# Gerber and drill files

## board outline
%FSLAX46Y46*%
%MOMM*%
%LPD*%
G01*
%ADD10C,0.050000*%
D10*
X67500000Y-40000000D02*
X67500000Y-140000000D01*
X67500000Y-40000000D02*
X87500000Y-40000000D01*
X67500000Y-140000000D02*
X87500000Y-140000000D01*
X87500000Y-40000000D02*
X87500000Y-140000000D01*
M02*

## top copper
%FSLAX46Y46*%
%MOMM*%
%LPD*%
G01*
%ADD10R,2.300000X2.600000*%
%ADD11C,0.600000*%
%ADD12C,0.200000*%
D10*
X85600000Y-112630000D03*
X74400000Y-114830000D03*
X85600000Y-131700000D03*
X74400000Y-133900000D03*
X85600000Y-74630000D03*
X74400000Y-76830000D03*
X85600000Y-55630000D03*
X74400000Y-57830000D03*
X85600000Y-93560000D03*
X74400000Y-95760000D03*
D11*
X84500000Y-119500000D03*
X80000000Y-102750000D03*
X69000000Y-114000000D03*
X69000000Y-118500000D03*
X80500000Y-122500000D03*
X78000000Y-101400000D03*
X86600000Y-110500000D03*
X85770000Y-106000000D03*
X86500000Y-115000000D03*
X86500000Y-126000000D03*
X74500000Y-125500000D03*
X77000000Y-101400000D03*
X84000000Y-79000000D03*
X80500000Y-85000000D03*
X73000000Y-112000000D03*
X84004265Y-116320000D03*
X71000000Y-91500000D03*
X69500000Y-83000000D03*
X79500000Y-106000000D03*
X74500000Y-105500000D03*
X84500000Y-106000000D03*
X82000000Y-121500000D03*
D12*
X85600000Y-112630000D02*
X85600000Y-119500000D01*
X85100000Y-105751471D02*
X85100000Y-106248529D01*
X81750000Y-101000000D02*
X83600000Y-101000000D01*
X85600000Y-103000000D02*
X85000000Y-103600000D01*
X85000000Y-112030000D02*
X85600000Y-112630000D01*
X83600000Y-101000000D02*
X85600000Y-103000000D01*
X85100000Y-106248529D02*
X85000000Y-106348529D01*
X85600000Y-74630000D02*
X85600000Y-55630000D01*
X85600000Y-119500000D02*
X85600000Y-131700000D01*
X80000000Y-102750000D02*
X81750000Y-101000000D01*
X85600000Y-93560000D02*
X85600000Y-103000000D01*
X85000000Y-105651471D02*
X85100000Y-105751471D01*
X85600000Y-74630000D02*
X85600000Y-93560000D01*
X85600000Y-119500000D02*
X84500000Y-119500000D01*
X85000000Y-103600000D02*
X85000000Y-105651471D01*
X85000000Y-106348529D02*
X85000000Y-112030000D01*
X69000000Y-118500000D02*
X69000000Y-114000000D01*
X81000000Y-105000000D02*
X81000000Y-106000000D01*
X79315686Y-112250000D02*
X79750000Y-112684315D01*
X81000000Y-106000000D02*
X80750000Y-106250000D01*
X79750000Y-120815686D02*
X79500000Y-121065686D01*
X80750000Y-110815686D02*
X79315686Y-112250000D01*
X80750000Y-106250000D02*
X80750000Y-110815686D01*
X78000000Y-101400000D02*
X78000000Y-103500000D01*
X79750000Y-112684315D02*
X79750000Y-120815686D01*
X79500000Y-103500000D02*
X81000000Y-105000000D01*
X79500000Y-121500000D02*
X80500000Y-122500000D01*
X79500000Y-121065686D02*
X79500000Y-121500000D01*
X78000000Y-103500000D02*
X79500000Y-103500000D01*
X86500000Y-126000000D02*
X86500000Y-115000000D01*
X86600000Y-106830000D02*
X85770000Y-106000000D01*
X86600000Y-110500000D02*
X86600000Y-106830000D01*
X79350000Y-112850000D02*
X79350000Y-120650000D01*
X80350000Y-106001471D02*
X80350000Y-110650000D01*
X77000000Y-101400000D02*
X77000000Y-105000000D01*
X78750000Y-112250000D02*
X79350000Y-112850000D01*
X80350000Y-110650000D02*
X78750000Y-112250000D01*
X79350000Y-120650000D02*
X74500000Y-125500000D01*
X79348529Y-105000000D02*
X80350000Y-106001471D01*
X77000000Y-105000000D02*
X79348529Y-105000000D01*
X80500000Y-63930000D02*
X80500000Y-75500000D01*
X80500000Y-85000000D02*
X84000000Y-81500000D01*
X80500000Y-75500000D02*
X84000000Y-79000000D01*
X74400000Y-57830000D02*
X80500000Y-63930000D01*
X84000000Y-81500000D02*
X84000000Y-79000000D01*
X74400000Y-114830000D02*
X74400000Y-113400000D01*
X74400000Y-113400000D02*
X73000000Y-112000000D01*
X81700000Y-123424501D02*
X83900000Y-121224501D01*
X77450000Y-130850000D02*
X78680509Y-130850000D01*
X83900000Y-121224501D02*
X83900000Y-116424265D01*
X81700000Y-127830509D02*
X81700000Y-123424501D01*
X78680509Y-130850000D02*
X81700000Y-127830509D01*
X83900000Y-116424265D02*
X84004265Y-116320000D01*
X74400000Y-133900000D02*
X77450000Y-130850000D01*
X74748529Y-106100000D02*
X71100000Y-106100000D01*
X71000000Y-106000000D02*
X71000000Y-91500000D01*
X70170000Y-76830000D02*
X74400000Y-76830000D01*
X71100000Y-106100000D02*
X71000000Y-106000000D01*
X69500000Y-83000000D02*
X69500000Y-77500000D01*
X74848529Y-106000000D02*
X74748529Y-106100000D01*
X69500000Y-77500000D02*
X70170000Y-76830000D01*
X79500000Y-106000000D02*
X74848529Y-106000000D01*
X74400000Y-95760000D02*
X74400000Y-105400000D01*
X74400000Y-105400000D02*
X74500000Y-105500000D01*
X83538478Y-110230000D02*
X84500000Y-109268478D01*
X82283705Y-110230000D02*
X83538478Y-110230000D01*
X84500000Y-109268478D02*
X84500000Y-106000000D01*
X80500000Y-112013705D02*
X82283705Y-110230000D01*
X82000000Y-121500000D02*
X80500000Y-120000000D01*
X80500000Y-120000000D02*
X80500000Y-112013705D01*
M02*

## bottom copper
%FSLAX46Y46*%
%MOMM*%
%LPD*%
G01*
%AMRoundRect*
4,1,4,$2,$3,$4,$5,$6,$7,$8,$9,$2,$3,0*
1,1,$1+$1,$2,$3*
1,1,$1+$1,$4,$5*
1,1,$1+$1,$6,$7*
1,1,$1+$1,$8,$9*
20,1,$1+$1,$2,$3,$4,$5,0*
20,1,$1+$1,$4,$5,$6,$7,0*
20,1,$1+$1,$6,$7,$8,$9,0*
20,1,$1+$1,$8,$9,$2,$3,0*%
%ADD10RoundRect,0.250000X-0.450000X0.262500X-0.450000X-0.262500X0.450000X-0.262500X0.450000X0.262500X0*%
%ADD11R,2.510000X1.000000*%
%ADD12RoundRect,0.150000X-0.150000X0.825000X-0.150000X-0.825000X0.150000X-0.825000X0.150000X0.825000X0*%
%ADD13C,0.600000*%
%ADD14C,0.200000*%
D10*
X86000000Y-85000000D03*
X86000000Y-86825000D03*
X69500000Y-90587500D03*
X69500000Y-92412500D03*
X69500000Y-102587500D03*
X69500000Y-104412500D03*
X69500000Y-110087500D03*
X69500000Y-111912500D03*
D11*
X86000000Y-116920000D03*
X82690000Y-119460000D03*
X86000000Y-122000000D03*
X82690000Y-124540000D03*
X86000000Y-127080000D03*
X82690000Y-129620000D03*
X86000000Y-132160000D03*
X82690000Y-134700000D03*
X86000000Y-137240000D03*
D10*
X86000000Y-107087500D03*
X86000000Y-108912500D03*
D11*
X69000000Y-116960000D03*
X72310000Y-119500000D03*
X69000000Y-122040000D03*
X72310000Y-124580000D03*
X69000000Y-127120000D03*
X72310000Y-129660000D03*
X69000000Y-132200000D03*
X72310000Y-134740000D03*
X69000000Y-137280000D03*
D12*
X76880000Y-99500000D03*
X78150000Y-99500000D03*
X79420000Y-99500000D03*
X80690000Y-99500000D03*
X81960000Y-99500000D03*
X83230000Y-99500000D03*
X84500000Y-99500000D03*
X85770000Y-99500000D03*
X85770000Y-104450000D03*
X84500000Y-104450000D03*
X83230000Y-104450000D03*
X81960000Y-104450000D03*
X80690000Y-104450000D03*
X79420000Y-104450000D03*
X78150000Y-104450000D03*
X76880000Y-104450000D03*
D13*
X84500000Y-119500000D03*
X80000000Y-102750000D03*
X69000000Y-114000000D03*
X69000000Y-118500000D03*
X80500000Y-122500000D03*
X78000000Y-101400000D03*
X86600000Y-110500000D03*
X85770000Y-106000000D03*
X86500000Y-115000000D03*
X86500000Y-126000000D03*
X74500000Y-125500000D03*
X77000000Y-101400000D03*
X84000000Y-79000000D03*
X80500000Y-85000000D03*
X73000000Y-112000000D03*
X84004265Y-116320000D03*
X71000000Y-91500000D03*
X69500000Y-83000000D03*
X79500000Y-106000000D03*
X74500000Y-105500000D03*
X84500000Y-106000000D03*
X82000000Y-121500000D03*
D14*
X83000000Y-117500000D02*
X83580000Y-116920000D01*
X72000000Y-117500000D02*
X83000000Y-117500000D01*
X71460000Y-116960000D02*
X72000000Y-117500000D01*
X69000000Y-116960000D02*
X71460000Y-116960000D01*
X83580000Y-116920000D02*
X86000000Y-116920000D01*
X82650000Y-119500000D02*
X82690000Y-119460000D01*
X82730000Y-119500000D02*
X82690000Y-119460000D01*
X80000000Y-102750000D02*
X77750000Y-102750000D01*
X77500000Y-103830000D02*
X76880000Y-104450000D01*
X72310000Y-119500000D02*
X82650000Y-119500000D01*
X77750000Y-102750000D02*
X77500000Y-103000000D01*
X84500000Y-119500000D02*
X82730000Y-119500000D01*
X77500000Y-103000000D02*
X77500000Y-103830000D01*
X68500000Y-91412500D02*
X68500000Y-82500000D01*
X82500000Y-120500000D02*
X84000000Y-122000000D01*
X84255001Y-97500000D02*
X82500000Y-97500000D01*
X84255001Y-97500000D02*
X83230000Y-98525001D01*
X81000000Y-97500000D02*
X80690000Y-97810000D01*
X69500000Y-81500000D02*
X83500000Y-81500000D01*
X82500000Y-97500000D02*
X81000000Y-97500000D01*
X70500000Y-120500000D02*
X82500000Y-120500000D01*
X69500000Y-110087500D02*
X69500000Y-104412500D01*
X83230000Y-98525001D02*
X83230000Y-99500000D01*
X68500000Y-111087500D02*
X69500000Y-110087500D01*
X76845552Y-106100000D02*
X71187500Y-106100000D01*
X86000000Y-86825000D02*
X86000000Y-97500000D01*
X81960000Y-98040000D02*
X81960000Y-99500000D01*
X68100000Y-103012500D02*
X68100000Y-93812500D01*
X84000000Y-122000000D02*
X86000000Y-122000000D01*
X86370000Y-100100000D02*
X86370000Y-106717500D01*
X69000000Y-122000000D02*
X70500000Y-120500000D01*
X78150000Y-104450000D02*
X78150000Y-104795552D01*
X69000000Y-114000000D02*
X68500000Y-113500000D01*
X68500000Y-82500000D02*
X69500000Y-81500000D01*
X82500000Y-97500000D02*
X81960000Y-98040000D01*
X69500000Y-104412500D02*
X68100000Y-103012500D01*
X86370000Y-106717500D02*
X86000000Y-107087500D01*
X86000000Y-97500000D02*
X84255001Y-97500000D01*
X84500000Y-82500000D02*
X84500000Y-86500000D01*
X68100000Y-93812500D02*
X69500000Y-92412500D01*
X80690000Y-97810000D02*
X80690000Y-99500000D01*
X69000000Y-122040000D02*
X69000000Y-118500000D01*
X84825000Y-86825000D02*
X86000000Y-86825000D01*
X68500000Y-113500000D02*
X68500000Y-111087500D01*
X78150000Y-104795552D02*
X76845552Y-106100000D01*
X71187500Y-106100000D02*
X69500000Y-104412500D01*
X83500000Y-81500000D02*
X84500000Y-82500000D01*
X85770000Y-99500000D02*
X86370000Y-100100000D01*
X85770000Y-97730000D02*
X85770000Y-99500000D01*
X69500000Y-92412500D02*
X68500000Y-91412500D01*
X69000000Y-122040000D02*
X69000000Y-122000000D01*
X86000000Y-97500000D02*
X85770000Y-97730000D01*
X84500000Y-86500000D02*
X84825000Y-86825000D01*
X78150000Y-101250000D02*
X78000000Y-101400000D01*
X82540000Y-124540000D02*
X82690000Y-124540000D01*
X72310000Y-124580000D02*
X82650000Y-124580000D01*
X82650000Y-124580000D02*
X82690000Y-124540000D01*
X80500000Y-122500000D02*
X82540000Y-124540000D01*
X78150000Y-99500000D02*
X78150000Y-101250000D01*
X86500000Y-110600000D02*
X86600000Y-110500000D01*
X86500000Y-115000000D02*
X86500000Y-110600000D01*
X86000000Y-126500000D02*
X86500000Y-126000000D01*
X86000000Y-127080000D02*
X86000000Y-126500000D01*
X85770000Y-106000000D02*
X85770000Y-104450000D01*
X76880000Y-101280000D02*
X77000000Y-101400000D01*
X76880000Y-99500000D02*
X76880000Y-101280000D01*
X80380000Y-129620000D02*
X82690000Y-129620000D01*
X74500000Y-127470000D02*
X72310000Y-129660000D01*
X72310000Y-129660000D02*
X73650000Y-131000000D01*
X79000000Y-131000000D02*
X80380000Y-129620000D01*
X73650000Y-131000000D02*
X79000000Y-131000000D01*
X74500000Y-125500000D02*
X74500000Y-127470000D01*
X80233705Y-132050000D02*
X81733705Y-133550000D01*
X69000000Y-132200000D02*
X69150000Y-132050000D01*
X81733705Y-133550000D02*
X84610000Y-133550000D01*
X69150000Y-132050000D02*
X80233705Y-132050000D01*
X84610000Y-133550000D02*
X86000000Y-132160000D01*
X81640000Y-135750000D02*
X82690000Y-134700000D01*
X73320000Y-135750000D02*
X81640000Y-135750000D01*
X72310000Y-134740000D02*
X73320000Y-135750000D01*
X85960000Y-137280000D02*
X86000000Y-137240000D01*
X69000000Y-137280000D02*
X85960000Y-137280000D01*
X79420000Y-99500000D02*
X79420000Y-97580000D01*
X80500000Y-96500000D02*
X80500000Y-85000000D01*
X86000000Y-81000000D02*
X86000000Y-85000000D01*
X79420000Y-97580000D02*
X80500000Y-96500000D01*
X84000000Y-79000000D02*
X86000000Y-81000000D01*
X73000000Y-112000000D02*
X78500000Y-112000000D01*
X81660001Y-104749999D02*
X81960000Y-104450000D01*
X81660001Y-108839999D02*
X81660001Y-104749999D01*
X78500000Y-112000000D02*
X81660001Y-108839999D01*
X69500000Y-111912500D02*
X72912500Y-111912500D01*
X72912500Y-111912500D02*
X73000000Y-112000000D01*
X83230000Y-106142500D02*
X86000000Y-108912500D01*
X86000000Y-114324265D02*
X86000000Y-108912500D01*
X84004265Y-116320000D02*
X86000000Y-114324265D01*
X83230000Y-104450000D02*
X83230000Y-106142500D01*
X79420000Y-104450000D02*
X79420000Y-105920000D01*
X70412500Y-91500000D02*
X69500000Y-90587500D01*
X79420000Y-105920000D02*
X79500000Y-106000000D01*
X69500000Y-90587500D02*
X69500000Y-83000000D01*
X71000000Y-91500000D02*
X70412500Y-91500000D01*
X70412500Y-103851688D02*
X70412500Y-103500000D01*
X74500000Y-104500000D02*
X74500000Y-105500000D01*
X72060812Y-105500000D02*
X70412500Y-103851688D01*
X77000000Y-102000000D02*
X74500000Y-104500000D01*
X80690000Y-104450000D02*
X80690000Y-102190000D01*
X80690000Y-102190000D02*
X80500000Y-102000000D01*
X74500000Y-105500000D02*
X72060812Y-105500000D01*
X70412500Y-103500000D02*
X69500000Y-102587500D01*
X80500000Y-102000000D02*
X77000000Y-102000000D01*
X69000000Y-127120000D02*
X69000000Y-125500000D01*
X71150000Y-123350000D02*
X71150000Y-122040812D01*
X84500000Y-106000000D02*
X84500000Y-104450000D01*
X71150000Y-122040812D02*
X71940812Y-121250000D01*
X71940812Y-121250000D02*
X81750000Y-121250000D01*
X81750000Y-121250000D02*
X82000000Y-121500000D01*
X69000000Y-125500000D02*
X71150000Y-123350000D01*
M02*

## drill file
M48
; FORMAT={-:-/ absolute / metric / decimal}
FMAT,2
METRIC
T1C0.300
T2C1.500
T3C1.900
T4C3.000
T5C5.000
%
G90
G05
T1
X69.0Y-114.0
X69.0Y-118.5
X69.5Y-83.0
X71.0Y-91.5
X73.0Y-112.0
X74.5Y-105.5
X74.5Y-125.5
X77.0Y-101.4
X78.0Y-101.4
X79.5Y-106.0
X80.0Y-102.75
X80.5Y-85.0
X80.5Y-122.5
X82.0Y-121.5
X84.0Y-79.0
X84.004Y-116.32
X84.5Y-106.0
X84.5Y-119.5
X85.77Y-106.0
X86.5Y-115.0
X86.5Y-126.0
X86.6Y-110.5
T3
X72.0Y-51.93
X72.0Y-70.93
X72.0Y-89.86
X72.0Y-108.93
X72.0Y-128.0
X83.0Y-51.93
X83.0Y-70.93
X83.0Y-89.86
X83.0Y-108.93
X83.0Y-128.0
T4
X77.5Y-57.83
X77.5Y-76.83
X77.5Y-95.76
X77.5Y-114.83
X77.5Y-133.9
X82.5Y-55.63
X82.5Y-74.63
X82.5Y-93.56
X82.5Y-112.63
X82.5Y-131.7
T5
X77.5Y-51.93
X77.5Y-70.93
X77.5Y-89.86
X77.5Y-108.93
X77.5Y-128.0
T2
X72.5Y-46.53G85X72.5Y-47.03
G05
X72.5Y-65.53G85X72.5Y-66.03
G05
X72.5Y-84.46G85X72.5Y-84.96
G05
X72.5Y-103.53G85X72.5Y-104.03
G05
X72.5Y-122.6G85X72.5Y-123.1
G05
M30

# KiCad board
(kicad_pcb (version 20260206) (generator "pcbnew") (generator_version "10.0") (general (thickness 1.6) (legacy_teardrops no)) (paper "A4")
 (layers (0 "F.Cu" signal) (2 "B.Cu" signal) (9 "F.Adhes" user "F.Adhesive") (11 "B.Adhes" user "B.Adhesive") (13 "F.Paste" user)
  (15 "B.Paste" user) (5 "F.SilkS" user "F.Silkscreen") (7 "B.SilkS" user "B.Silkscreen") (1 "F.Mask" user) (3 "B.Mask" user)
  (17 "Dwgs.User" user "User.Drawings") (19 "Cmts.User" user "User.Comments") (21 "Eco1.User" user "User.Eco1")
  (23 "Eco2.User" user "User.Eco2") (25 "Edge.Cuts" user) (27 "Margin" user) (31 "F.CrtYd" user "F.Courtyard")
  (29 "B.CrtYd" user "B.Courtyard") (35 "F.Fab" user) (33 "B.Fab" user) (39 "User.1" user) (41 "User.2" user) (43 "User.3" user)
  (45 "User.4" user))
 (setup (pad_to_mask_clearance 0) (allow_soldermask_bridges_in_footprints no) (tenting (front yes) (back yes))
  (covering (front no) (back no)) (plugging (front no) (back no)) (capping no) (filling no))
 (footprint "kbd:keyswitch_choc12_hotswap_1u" (layer "F.Cu") (at 77.5 108.93)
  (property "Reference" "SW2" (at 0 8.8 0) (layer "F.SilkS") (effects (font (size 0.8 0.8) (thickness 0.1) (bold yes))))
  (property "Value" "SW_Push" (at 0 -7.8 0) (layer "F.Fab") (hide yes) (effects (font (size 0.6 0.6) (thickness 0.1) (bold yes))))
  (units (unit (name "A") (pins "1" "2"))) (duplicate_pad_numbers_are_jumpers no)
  (pad "" np_thru_hole circle (at -5.5 0 270) (size 1.9 1.9) (drill 1.9) (layers "*.Cu" "*.Mask"))
  (pad "" np_thru_hole oval (at -5 -5.15) (size 1.5 2) (drill oval 1.5 2) (layers "*.Cu" "*.Mask"))
  (pad "" np_thru_hole circle (at 0 0 270) (size 5 5) (drill 5) (layers "*.Cu" "*.Mask"))
  (pad "" np_thru_hole circle (at 0 5.9 270) (size 3 3) (drill 3) (layers "*.Cu" "*.Mask"))
  (pad "" np_thru_hole circle (at 5 3.7 270) (size 3 3) (drill 3) (layers "*.Cu" "*.Mask"))
  (pad "" np_thru_hole circle (at 5.5 0 270) (size 1.9 1.9) (drill 1.9) (layers "*.Cu" "*.Mask"))
  (pad "1" smd rect (at 8.1 3.7 180) (size 2.3 2.6) (layers "F.Cu" "F.Mask" "F.Paste") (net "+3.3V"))
  (pad "2" smd rect (at -3.1 5.9 180) (size 2.3 2.6) (layers "F.Cu" "F.Mask" "F.Paste") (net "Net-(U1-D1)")))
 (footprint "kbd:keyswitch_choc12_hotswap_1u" (layer "F.Cu") (at 77.5 128)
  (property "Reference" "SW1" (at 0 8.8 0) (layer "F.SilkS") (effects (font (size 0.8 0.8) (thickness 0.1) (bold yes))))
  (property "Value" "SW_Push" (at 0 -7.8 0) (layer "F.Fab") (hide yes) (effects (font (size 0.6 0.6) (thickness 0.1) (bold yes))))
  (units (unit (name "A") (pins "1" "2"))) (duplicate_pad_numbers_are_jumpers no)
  (pad "" np_thru_hole circle (at -5.5 0 270) (size 1.9 1.9) (drill 1.9) (layers "*.Cu" "*.Mask"))
  (pad "" np_thru_hole oval (at -5 -5.15) (size 1.5 2) (drill oval 1.5 2) (layers "*.Cu" "*.Mask"))
  (pad "" np_thru_hole circle (at 0 0 270) (size 5 5) (drill 5) (layers "*.Cu" "*.Mask"))
  (pad "" np_thru_hole circle (at 0 5.9 270) (size 3 3) (drill 3) (layers "*.Cu" "*.Mask"))
  (pad "" np_thru_hole circle (at 5 3.7 270) (size 3 3) (drill 3) (layers "*.Cu" "*.Mask"))
  (pad "" np_thru_hole circle (at 5.5 0 270) (size 1.9 1.9) (drill 1.9) (layers "*.Cu" "*.Mask"))
  (pad "1" smd rect (at 8.1 3.7 180) (size 2.3 2.6) (layers "F.Cu" "F.Mask" "F.Paste") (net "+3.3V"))
  (pad "2" smd rect (at -3.1 5.9 180) (size 2.3 2.6) (layers "F.Cu" "F.Mask" "F.Paste") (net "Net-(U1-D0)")))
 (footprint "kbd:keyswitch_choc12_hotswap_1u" (layer "F.Cu") (at 77.5 70.93)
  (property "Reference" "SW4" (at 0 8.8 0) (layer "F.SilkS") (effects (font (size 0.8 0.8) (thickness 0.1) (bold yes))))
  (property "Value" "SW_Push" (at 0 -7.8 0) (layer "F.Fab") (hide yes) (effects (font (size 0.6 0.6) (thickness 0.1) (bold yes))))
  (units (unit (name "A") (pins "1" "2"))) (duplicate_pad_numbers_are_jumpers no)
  (pad "" np_thru_hole circle (at -5.5 0 270) (size 1.9 1.9) (drill 1.9) (layers "*.Cu" "*.Mask"))
  (pad "" np_thru_hole oval (at -5 -5.15) (size 1.5 2) (drill oval 1.5 2) (layers "*.Cu" "*.Mask"))
  (pad "" np_thru_hole circle (at 0 0 270) (size 5 5) (drill 5) (layers "*.Cu" "*.Mask"))
  (pad "" np_thru_hole circle (at 0 5.9 270) (size 3 3) (drill 3) (layers "*.Cu" "*.Mask"))
  (pad "" np_thru_hole circle (at 5 3.7 270) (size 3 3) (drill 3) (layers "*.Cu" "*.Mask"))
  (pad "" np_thru_hole circle (at 5.5 0 270) (size 1.9 1.9) (drill 1.9) (layers "*.Cu" "*.Mask"))
  (pad "1" smd rect (at 8.1 3.7 180) (size 2.3 2.6) (layers "F.Cu" "F.Mask" "F.Paste") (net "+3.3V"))
  (pad "2" smd rect (at -3.1 5.9 180) (size 2.3 2.6) (layers "F.Cu" "F.Mask" "F.Paste") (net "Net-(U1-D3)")))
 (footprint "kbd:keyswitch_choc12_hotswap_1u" (layer "F.Cu") (at 77.5 51.93)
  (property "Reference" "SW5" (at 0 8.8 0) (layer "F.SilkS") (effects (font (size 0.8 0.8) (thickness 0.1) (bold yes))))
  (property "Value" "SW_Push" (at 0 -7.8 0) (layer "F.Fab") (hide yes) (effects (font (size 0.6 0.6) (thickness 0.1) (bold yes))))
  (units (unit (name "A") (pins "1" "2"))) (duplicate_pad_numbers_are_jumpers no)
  (pad "" np_thru_hole circle (at -5.5 0 270) (size 1.9 1.9) (drill 1.9) (layers "*.Cu" "*.Mask"))
  (pad "" np_thru_hole oval (at -5 -5.15) (size 1.5 2) (drill oval 1.5 2) (layers "*.Cu" "*.Mask"))
  (pad "" np_thru_hole circle (at 0 0 270) (size 5 5) (drill 5) (layers "*.Cu" "*.Mask"))
  (pad "" np_thru_hole circle (at 0 5.9 270) (size 3 3) (drill 3) (layers "*.Cu" "*.Mask"))
  (pad "" np_thru_hole circle (at 5 3.7 270) (size 3 3) (drill 3) (layers "*.Cu" "*.Mask"))
  (pad "" np_thru_hole circle (at 5.5 0 270) (size 1.9 1.9) (drill 1.9) (layers "*.Cu" "*.Mask"))
  (pad "1" smd rect (at 8.1 3.7 180) (size 2.3 2.6) (layers "F.Cu" "F.Mask" "F.Paste") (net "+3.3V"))
  (pad "2" smd rect (at -3.1 5.9 180) (size 2.3 2.6) (layers "F.Cu" "F.Mask" "F.Paste") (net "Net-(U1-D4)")))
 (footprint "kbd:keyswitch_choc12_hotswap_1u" (layer "F.Cu") (at 77.5 89.86)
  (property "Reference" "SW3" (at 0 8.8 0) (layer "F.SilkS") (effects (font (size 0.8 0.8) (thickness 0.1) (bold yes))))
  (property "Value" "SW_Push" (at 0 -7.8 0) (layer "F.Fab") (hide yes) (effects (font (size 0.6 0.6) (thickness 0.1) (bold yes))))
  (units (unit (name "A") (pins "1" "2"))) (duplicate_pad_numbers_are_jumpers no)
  (pad "" np_thru_hole circle (at -5.5 0 270) (size 1.9 1.9) (drill 1.9) (layers "*.Cu" "*.Mask"))
  (pad "" np_thru_hole oval (at -5 -5.15) (size 1.5 2) (drill oval 1.5 2) (layers "*.Cu" "*.Mask"))
  (pad "" np_thru_hole circle (at 0 0 270) (size 5 5) (drill 5) (layers "*.Cu" "*.Mask"))
  (pad "" np_thru_hole circle (at 0 5.9 270) (size 3 3) (drill 3) (layers "*.Cu" "*.Mask"))
  (pad "" np_thru_hole circle (at 5 3.7 270) (size 3 3) (drill 3) (layers "*.Cu" "*.Mask"))
  (pad "" np_thru_hole circle (at 5.5 0 270) (size 1.9 1.9) (drill 1.9) (layers "*.Cu" "*.Mask"))
  (pad "1" smd rect (at 8.1 3.7 180) (size 2.3 2.6) (layers "F.Cu" "F.Mask" "F.Paste") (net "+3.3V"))
  (pad "2" smd rect (at -3.1 5.9 180) (size 2.3 2.6) (layers "F.Cu" "F.Mask" "F.Paste") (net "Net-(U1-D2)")))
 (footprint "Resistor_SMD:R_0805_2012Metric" (layer "B.Cu") (at 86 85.9125 -90)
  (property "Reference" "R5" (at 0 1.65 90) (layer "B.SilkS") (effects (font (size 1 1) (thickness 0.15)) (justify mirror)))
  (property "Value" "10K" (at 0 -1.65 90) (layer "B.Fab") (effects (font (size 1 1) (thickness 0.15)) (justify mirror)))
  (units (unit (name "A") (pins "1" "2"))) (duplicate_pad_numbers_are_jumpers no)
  (pad "1" smd roundrect (at -0.9125 0 270) (size 1.025 1.4) (layers "B.Cu" "B.Mask" "B.Paste") (roundrect_rratio 0.243902)
   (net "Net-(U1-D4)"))
  (pad "2" smd roundrect (at 0.9125 0 270) (size 1.025 1.4) (layers "B.Cu" "B.Mask" "B.Paste") (roundrect_rratio 0.243902) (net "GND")))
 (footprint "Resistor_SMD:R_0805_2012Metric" (layer "B.Cu") (at 69.5 91.5 -90)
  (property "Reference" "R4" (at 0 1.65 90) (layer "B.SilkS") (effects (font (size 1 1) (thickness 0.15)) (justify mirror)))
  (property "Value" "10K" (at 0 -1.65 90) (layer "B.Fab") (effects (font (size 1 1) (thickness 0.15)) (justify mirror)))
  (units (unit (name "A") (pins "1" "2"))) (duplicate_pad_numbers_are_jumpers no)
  (pad "1" smd roundrect (at -0.9125 0 270) (size 1.025 1.4) (layers "B.Cu" "B.Mask" "B.Paste") (roundrect_rratio 0.243902)
   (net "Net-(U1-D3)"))
  (pad "2" smd roundrect (at 0.9125 0 270) (size 1.025 1.4) (layers "B.Cu" "B.Mask" "B.Paste") (roundrect_rratio 0.243902) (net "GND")))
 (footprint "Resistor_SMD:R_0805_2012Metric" (layer "B.Cu") (at 69.5 103.5 -90)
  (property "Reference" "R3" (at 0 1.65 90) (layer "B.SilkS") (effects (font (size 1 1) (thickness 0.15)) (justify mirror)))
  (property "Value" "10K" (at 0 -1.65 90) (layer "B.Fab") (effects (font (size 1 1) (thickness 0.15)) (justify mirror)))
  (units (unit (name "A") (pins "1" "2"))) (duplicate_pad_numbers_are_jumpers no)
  (pad "1" smd roundrect (at -0.9125 0 270) (size 1.025 1.4) (layers "B.Cu" "B.Mask" "B.Paste") (roundrect_rratio 0.243902)
   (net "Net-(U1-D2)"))
  (pad "2" smd roundrect (at 0.9125 0 270) (size 1.025 1.4) (layers "B.Cu" "B.Mask" "B.Paste") (roundrect_rratio 0.243902) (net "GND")))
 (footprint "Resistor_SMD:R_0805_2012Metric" (layer "B.Cu") (at 69.5 111 -90)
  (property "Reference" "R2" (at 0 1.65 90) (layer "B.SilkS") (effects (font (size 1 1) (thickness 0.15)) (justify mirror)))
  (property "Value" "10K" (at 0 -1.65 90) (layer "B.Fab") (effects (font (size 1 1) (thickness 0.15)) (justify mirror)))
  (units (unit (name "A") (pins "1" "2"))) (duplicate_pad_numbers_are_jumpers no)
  (pad "1" smd roundrect (at -0.9125 0 270) (size 1.025 1.4) (layers "B.Cu" "B.Mask" "B.Paste") (roundrect_rratio 0.243902) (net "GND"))
  (pad "2" smd roundrect (at 0.9125 0 270) (size 1.025 1.4) (layers "B.Cu" "B.Mask" "B.Paste") (roundrect_rratio 0.243902)
   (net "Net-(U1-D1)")))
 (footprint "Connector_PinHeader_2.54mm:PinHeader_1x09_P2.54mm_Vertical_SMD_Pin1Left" (layer "B.Cu") (at 84.345 127.08 180)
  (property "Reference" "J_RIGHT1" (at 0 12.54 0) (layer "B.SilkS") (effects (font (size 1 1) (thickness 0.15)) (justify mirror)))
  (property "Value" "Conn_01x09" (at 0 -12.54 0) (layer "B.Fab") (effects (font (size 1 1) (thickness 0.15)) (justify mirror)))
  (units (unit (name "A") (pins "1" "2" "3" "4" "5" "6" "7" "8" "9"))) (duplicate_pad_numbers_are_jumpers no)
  (pad "1" smd rect (at -1.655 10.16 180) (size 2.51 1) (layers "B.Cu" "B.Mask" "B.Paste") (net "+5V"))
  (pad "2" smd rect (at 1.655 7.62 180) (size 2.51 1) (layers "B.Cu" "B.Mask" "B.Paste") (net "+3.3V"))
  (pad "3" smd rect (at -1.655 5.08 180) (size 2.51 1) (layers "B.Cu" "B.Mask" "B.Paste") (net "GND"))
  (pad "4" smd rect (at 1.655 2.54 180) (size 2.51 1) (layers "B.Cu" "B.Mask" "B.Paste") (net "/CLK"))
  (pad "5" smd rect (at -1.655 0 180) (size 2.51 1) (layers "B.Cu" "B.Mask" "B.Paste") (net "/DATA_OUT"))
  (pad "6" smd rect (at 1.655 -2.54 180) (size 2.51 1) (layers "B.Cu" "B.Mask" "B.Paste") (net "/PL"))
  (pad "7" smd rect (at -1.655 -5.08 180) (size 2.51 1) (layers "B.Cu" "B.Mask" "B.Paste") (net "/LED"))
  (pad "8" smd rect (at 1.655 -7.62 180) (size 2.51 1) (layers "B.Cu" "B.Mask" "B.Paste") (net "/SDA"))
  (pad "9" smd rect (at -1.655 -10.16 180) (size 2.51 1) (layers "B.Cu" "B.Mask" "B.Paste") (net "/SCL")))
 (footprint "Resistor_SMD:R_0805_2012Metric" (layer "B.Cu") (at 86 108 -90)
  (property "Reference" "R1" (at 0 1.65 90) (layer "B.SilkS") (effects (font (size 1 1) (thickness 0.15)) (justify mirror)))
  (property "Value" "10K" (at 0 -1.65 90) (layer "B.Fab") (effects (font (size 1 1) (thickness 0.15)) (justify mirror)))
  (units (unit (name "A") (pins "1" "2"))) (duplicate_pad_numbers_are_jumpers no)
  (pad "1" smd roundrect (at -0.9125 0 270) (size 1.025 1.4) (layers "B.Cu" "B.Mask" "B.Paste") (roundrect_rratio 0.243902) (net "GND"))
  (pad "2" smd roundrect (at 0.9125 0 270) (size 1.025 1.4) (layers "B.Cu" "B.Mask" "B.Paste") (roundrect_rratio 0.243902)
   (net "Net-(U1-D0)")))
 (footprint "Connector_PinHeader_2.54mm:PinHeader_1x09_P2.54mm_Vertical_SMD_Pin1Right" (layer "B.Cu") (at 70.655 127.12 180)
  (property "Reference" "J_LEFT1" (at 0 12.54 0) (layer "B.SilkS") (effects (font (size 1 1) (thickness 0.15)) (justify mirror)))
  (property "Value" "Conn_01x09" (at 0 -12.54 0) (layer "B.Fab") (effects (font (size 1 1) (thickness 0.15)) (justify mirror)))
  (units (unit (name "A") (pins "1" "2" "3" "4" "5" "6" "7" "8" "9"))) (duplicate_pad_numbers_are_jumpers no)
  (pad "1" smd rect (at 1.655 10.16 180) (size 2.51 1) (layers "B.Cu" "B.Mask" "B.Paste") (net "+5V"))
  (pad "2" smd rect (at -1.655 7.62 180) (size 2.51 1) (layers "B.Cu" "B.Mask" "B.Paste") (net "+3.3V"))
  (pad "3" smd rect (at 1.655 5.08 180) (size 2.51 1) (layers "B.Cu" "B.Mask" "B.Paste") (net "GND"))
  (pad "4" smd rect (at -1.655 2.54 180) (size 2.51 1) (layers "B.Cu" "B.Mask" "B.Paste") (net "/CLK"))
  (pad "5" smd rect (at 1.655 0 180) (size 2.51 1) (layers "B.Cu" "B.Mask" "B.Paste") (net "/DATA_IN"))
  (pad "6" smd rect (at -1.655 -2.54 180) (size 2.51 1) (layers "B.Cu" "B.Mask" "B.Paste") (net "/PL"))
  (pad "7" smd rect (at 1.655 -5.08 180) (size 2.51 1) (layers "B.Cu" "B.Mask" "B.Paste") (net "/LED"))
  (pad "8" smd rect (at -1.655 -7.62 180) (size 2.51 1) (layers "B.Cu" "B.Mask" "B.Paste") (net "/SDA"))
  (pad "9" smd rect (at 1.655 -10.16 180) (size 2.51 1) (layers "B.Cu" "B.Mask" "B.Paste") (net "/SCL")))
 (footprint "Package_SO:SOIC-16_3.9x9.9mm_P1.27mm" (layer "B.Cu") (at 81.325 101.975 -90)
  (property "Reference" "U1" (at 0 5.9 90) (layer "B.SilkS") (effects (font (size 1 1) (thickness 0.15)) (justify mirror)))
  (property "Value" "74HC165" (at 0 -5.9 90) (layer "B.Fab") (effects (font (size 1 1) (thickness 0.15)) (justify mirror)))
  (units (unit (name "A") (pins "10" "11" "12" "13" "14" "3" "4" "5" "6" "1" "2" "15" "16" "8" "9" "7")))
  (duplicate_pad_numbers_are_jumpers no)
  (pad "1" smd roundrect (at -2.475 4.445 270) (size 1.95 0.6) (layers "B.Cu" "B.Mask" "B.Paste") (roundrect_rratio 0.25) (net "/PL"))
  (pad "2" smd roundrect (at -2.475 3.175 270) (size 1.95 0.6) (layers "B.Cu" "B.Mask" "B.Paste") (roundrect_rratio 0.25) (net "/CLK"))
  (pad "3" smd roundrect (at -2.475 1.905 270) (size 1.95 0.6) (layers "B.Cu" "B.Mask" "B.Paste") (roundrect_rratio 0.25)
   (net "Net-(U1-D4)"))
  (pad "4" smd roundrect (at -2.475 0.635 270) (size 1.95 0.6) (layers "B.Cu" "B.Mask" "B.Paste") (roundrect_rratio 0.25) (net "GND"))
  (pad "5" smd roundrect (at -2.475 -0.635 270) (size 1.95 0.6) (layers "B.Cu" "B.Mask" "B.Paste") (roundrect_rratio 0.25) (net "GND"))
  (pad "6" smd roundrect (at -2.475 -1.905 270) (size 1.95 0.6) (layers "B.Cu" "B.Mask" "B.Paste") (roundrect_rratio 0.25) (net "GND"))
  (pad "7" smd roundrect (at -2.475 -3.175 270) (size 1.95 0.6) (layers "B.Cu" "B.Mask" "B.Paste") (roundrect_rratio 0.25)
   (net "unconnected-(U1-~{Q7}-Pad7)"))
  (pad "8" smd roundrect (at -2.475 -4.445 270) (size 1.95 0.6) (layers "B.Cu" "B.Mask" "B.Paste") (roundrect_rratio 0.25) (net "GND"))
  (pad "9" smd roundrect (at 2.475 -4.445 270) (size 1.95 0.6) (layers "B.Cu" "B.Mask" "B.Paste") (roundrect_rratio 0.25) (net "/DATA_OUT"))
  (pad "10" smd roundrect (at 2.475 -3.175 270) (size 1.95 0.6) (layers "B.Cu" "B.Mask" "B.Paste") (roundrect_rratio 0.25) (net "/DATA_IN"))
  (pad "11" smd roundrect (at 2.475 -1.905 270) (size 1.95 0.6) (layers "B.Cu" "B.Mask" "B.Paste") (roundrect_rratio 0.25)
   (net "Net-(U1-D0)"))
  (pad "12" smd roundrect (at 2.475 -0.635 270) (size 1.95 0.6) (layers "B.Cu" "B.Mask" "B.Paste") (roundrect_rratio 0.25)
   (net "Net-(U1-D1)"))
  (pad "13" smd roundrect (at 2.475 0.635 270) (size 1.95 0.6) (layers "B.Cu" "B.Mask" "B.Paste") (roundrect_rratio 0.25)
   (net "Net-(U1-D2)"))
  (pad "14" smd roundrect (at 2.475 1.905 270) (size 1.95 0.6) (layers "B.Cu" "B.Mask" "B.Paste") (roundrect_rratio 0.25)
   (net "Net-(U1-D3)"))
  (pad "15" smd roundrect (at 2.475 3.175 270) (size 1.95 0.6) (layers "B.Cu" "B.Mask" "B.Paste") (roundrect_rratio 0.25) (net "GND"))
  (pad "16" smd roundrect (at 2.475 4.445 270) (size 1.95 0.6) (layers "B.Cu" "B.Mask" "B.Paste") (roundrect_rratio 0.25) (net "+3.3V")))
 (gr_line (start 67.5 40) (end 67.5 140) (stroke (width 0.05) (type default)) (layer "Edge.Cuts"))
 (gr_line (start 67.5 40) (end 87.5 40) (stroke (width 0.05) (type default)) (layer "Edge.Cuts"))
 (gr_line (start 67.5 140) (end 87.5 140) (stroke (width 0.05) (type default)) (layer "Edge.Cuts"))
 (gr_line (start 87.5 40) (end 87.5 140) (stroke (width 0.05) (type default)) (layer "Edge.Cuts"))
 (segment (start 83 117.5) (end 83.58 116.92) (width 0.2) (layer "B.Cu") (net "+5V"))
 (segment (start 72 117.5) (end 83 117.5) (width 0.2) (layer "B.Cu") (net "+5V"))
 (segment (start 71.46 116.96) (end 72 117.5) (width 0.2) (layer "B.Cu") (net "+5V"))
 (segment (start 69 116.96) (end 71.46 116.96) (width 0.2) (layer "B.Cu") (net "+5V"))
 (segment (start 83.58 116.92) (end 86 116.92) (width 0.2) (layer "B.Cu") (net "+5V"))
 (segment (start 85.6 112.63) (end 85.6 119.5) (width 0.2) (layer "F.Cu") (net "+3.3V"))
 (segment (start 85.1 105.751471) (end 85.1 106.248529) (width 0.2) (layer "F.Cu") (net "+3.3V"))
 (segment (start 81.75 101) (end 83.6 101) (width 0.2) (layer "F.Cu") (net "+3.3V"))
 (segment (start 85.6 103) (end 85 103.6) (width 0.2) (layer "F.Cu") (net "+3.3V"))
 (segment (start 85 112.03) (end 85.6 112.63) (width 0.2) (layer "F.Cu") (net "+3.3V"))
 (segment (start 83.6 101) (end 85.6 103) (width 0.2) (layer "F.Cu") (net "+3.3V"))
 (segment (start 85.1 106.248529) (end 85 106.348529) (width 0.2) (layer "F.Cu") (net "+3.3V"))
 (segment (start 85.6 74.63) (end 85.6 55.63) (width 0.2) (layer "F.Cu") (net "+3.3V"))
 (segment (start 85.6 119.5) (end 85.6 131.7) (width 0.2) (layer "F.Cu") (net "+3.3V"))
 (segment (start 80 102.75) (end 81.75 101) (width 0.2) (layer "F.Cu") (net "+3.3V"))
 (segment (start 85.6 93.56) (end 85.6 103) (width 0.2) (layer "F.Cu") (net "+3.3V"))
 (segment (start 85 105.651471) (end 85.1 105.751471) (width 0.2) (layer "F.Cu") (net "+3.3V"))
 (segment (start 85.6 74.63) (end 85.6 93.56) (width 0.2) (layer "F.Cu") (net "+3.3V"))
 (segment (start 85.6 119.5) (end 84.5 119.5) (width 0.2) (layer "F.Cu") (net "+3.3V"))
 (segment (start 85 103.6) (end 85 105.651471) (width 0.2) (layer "F.Cu") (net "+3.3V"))
 (segment (start 85 106.348529) (end 85 112.03) (width 0.2) (layer "F.Cu") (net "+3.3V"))
 (via (at 84.5 119.5) (size 0.6) (drill 0.3) (layers "F.Cu" "B.Cu") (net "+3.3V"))
 (via (at 80 102.75) (size 0.6) (drill 0.3) (layers "F.Cu" "B.Cu") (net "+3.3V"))
 (segment (start 82.65 119.5) (end 82.69 119.46) (width 0.2) (layer "B.Cu") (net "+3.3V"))
 (segment (start 82.73 119.5) (end 82.69 119.46) (width 0.2) (layer "B.Cu") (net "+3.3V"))
 (segment (start 80 102.75) (end 77.75 102.75) (width 0.2) (layer "B.Cu") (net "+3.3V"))
 (segment (start 77.5 103.83) (end 76.88 104.45) (width 0.2) (layer "B.Cu") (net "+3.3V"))
 (segment (start 72.31 119.5) (end 82.65 119.5) (width 0.2) (layer "B.Cu") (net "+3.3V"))
 (segment (start 77.75 102.75) (end 77.5 103) (width 0.2) (layer "B.Cu") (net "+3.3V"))
 (segment (start 84.5 119.5) (end 82.73 119.5) (width 0.2) (layer "B.Cu") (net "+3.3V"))
 (segment (start 77.5 103) (end 77.5 103.83) (width 0.2) (layer "B.Cu") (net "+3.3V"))
 (segment (start 69 118.5) (end 69 114) (width 0.2) (layer "F.Cu") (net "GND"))
 (via (at 69 114) (size 0.6) (drill 0.3) (layers "F.Cu" "B.Cu") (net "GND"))
 (via (at 69 118.5) (size 0.6) (drill 0.3) (layers "F.Cu" "B.Cu") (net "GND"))
 (segment (start 68.5 91.4125) (end 68.5 82.5) (width 0.2) (layer "B.Cu") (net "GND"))
 (segment (start 82.5 120.5) (end 84 122) (width 0.2) (layer "B.Cu") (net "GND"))
 (segment (start 84.255001 97.5) (end 82.5 97.5) (width 0.2) (layer "B.Cu") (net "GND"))
 (segment (start 84.255001 97.5) (end 83.23 98.525001) (width 0.2) (layer "B.Cu") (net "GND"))
 (segment (start 81 97.5) (end 80.69 97.81) (width 0.2) (layer "B.Cu") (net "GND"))
 (segment (start 69.5 81.5) (end 83.5 81.5) (width 0.2) (layer "B.Cu") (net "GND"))
 (segment (start 82.5 97.5) (end 81 97.5) (width 0.2) (layer "B.Cu") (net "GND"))
 (segment (start 70.5 120.5) (end 82.5 120.5) (width 0.2) (layer "B.Cu") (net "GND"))
 (segment (start 69.5 110.0875) (end 69.5 104.4125) (width 0.2) (layer "B.Cu") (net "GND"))
 (segment (start 83.23 98.525001) (end 83.23 99.5) (width 0.2) (layer "B.Cu") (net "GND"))
 (segment (start 68.5 111.0875) (end 69.5 110.0875) (width 0.2) (layer "B.Cu") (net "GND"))
 (segment (start 76.845552 106.1) (end 71.1875 106.1) (width 0.2) (layer "B.Cu") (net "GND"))
 (segment (start 86 86.825) (end 86 97.5) (width 0.2) (layer "B.Cu") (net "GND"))
 (segment (start 81.96 98.04) (end 81.96 99.5) (width 0.2) (layer "B.Cu") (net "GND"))
 (segment (start 68.1 103.0125) (end 68.1 93.8125) (width 0.2) (layer "B.Cu") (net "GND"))
 (segment (start 84 122) (end 86 122) (width 0.2) (layer "B.Cu") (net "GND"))
 (segment (start 86.37 100.1) (end 86.37 106.7175) (width 0.2) (layer "B.Cu") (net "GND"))
 (segment (start 69 122) (end 70.5 120.5) (width 0.2) (layer "B.Cu") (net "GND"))
 (segment (start 78.15 104.45) (end 78.15 104.795552) (width 0.2) (layer "B.Cu") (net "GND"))
 (segment (start 69 114) (end 68.5 113.5) (width 0.2) (layer "B.Cu") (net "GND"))
 (segment (start 68.5 82.5) (end 69.5 81.5) (width 0.2) (layer "B.Cu") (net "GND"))
 (segment (start 82.5 97.5) (end 81.96 98.04) (width 0.2) (layer "B.Cu") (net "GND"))
 (segment (start 69.5 104.4125) (end 68.1 103.0125) (width 0.2) (layer "B.Cu") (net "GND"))
 (segment (start 86.37 106.7175) (end 86 107.0875) (width 0.2) (layer "B.Cu") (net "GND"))
 (segment (start 86 97.5) (end 84.255001 97.5) (width 0.2) (layer "B.Cu") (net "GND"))
 (segment (start 84.5 82.5) (end 84.5 86.5) (width 0.2) (layer "B.Cu") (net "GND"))
 (segment (start 68.1 93.8125) (end 69.5 92.4125) (width 0.2) (layer "B.Cu") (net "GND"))
 (segment (start 80.69 97.81) (end 80.69 99.5) (width 0.2) (layer "B.Cu") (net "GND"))
 (segment (start 69 122.04) (end 69 118.5) (width 0.2) (layer "B.Cu") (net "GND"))
 (segment (start 84.825 86.825) (end 86 86.825) (width 0.2) (layer "B.Cu") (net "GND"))
 (segment (start 68.5 113.5) (end 68.5 111.0875) (width 0.2) (layer "B.Cu") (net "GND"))
 (segment (start 78.15 104.795552) (end 76.845552 106.1) (width 0.2) (layer "B.Cu") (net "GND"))
 (segment (start 71.1875 106.1) (end 69.5 104.4125) (width 0.2) (layer "B.Cu") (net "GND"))
 (segment (start 83.5 81.5) (end 84.5 82.5) (width 0.2) (layer "B.Cu") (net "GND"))
 (segment (start 85.77 99.5) (end 86.37 100.1) (width 0.2) (layer "B.Cu") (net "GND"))
 (segment (start 85.77 97.73) (end 85.77 99.5) (width 0.2) (layer "B.Cu") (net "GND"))
 (segment (start 69.5 92.4125) (end 68.5 91.4125) (width 0.2) (layer "B.Cu") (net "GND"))
 (segment (start 69 122.04) (end 69 122) (width 0.2) (layer "B.Cu") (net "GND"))
 (segment (start 86 97.5) (end 85.77 97.73) (width 0.2) (layer "B.Cu") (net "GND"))
 (segment (start 84.5 86.5) (end 84.825 86.825) (width 0.2) (layer "B.Cu") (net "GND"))
 (segment (start 81 105) (end 81 106) (width 0.2) (layer "F.Cu") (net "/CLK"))
 (segment (start 79.315686 112.25) (end 79.75 112.684315) (width 0.2) (layer "F.Cu") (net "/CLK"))
 (segment (start 81 106) (end 80.75 106.25) (width 0.2) (layer "F.Cu") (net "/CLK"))
 (segment (start 79.75 120.815686) (end 79.5 121.065686) (width 0.2) (layer "F.Cu") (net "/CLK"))
 (segment (start 80.75 110.815686) (end 79.315686 112.25) (width 0.2) (layer "F.Cu") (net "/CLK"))
 (segment (start 80.75 106.25) (end 80.75 110.815686) (width 0.2) (layer "F.Cu") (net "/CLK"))
 (segment (start 78 101.4) (end 78 103.5) (width 0.2) (layer "F.Cu") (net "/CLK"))
 (segment (start 79.75 112.684315) (end 79.75 120.815686) (width 0.2) (layer "F.Cu") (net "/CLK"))
 (segment (start 79.5 103.5) (end 81 105) (width 0.2) (layer "F.Cu") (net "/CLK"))
 (segment (start 79.5 121.5) (end 80.5 122.5) (width 0.2) (layer "F.Cu") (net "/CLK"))
 (segment (start 79.5 121.065686) (end 79.5 121.5) (width 0.2) (layer "F.Cu") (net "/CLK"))
 (segment (start 78 103.5) (end 79.5 103.5) (width 0.2) (layer "F.Cu") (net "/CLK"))
 (via (at 80.5 122.5) (size 0.6) (drill 0.3) (layers "F.Cu" "B.Cu") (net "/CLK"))
 (via (at 78 101.4) (size 0.6) (drill 0.3) (layers "F.Cu" "B.Cu") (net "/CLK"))
 (segment (start 78.15 101.25) (end 78 101.4) (width 0.2) (layer "B.Cu") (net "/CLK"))
 (segment (start 82.54 124.54) (end 82.69 124.54) (width 0.2) (layer "B.Cu") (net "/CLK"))
 (segment (start 72.31 124.58) (end 82.65 124.58) (width 0.2) (layer "B.Cu") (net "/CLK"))
 (segment (start 82.65 124.58) (end 82.69 124.54) (width 0.2) (layer "B.Cu") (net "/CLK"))
 (segment (start 80.5 122.5) (end 82.54 124.54) (width 0.2) (layer "B.Cu") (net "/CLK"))
 (segment (start 78.15 99.5) (end 78.15 101.25) (width 0.2) (layer "B.Cu") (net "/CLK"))
 (segment (start 86.5 126) (end 86.5 115) (width 0.2) (layer "F.Cu") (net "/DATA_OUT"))
 (segment (start 86.6 106.83) (end 85.77 106) (width 0.2) (layer "F.Cu") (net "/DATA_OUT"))
 (segment (start 86.6 110.5) (end 86.6 106.83) (width 0.2) (layer "F.Cu") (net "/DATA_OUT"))
 (via (at 86.6 110.5) (size 0.6) (drill 0.3) (layers "F.Cu" "B.Cu") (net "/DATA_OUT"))
 (via (at 85.77 106) (size 0.6) (drill 0.3) (layers "F.Cu" "B.Cu") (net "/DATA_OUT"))
 (via (at 86.5 115) (size 0.6) (drill 0.3) (layers "F.Cu" "B.Cu") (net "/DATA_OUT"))
 (via (at 86.5 126) (size 0.6) (drill 0.3) (layers "F.Cu" "B.Cu") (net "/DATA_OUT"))
 (segment (start 86.5 110.6) (end 86.6 110.5) (width 0.2) (layer "B.Cu") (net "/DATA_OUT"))
 (segment (start 86.5 115) (end 86.5 110.6) (width 0.2) (layer "B.Cu") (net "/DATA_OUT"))
 (segment (start 86 126.5) (end 86.5 126) (width 0.2) (layer "B.Cu") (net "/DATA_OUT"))
 (segment (start 86 127.08) (end 86 126.5) (width 0.2) (layer "B.Cu") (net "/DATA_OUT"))
 (segment (start 85.77 106) (end 85.77 104.45) (width 0.2) (layer "B.Cu") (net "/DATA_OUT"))
 (segment (start 79.35 112.85) (end 79.35 120.65) (width 0.2) (layer "F.Cu") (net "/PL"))
 (segment (start 80.35 106.001471) (end 80.35 110.65) (width 0.2) (layer "F.Cu") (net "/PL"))
 (segment (start 77 101.4) (end 77 105) (width 0.2) (layer "F.Cu") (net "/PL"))
 (segment (start 78.75 112.25) (end 79.35 112.85) (width 0.2) (layer "F.Cu") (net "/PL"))
 (segment (start 80.35 110.65) (end 78.75 112.25) (width 0.2) (layer "F.Cu") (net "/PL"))
 (segment (start 79.35 120.65) (end 74.5 125.5) (width 0.2) (layer "F.Cu") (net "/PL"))
 (segment (start 79.348529 105) (end 80.35 106.001471) (width 0.2) (layer "F.Cu") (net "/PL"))
 (segment (start 77 105) (end 79.348529 105) (width 0.2) (layer "F.Cu") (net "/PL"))
 (via (at 74.5 125.5) (size 0.6) (drill 0.3) (layers "F.Cu" "B.Cu") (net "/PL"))
 (via (at 77 101.4) (size 0.6) (drill 0.3) (layers "F.Cu" "B.Cu") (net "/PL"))
 (segment (start 76.88 101.28) (end 77 101.4) (width 0.2) (layer "B.Cu") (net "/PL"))
 (segment (start 76.88 99.5) (end 76.88 101.28) (width 0.2) (layer "B.Cu") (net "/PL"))
 (segment (start 80.38 129.62) (end 82.69 129.62) (width 0.2) (layer "B.Cu") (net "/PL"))
 (segment (start 74.5 127.47) (end 72.31 129.66) (width 0.2) (layer "B.Cu") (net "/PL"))
 (segment (start 72.31 129.66) (end 73.65 131) (width 0.2) (layer "B.Cu") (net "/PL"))
 (segment (start 79 131) (end 80.38 129.62) (width 0.2) (layer "B.Cu") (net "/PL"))
 (segment (start 73.65 131) (end 79 131) (width 0.2) (layer "B.Cu") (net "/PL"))
 (segment (start 74.5 125.5) (end 74.5 127.47) (width 0.2) (layer "B.Cu") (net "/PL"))
 (segment (start 80.233705 132.05) (end 81.733705 133.55) (width 0.2) (layer "B.Cu") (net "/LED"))
 (segment (start 69 132.2) (end 69.15 132.05) (width 0.2) (layer "B.Cu") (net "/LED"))
 (segment (start 81.733705 133.55) (end 84.61 133.55) (width 0.2) (layer "B.Cu") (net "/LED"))
 (segment (start 69.15 132.05) (end 80.233705 132.05) (width 0.2) (layer "B.Cu") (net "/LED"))
 (segment (start 84.61 133.55) (end 86 132.16) (width 0.2) (layer "B.Cu") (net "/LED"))
 (segment (start 81.64 135.75) (end 82.69 134.7) (width 0.2) (layer "B.Cu") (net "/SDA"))
 (segment (start 73.32 135.75) (end 81.64 135.75) (width 0.2) (layer "B.Cu") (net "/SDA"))
 (segment (start 72.31 134.74) (end 73.32 135.75) (width 0.2) (layer "B.Cu") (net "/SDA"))
 (segment (start 85.96 137.28) (end 86 137.24) (width 0.2) (layer "B.Cu") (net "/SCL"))
 (segment (start 69 137.28) (end 85.96 137.28) (width 0.2) (layer "B.Cu") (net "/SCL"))
 (segment (start 80.5 63.93) (end 80.5 75.5) (width 0.2) (layer "F.Cu") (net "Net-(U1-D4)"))
 (segment (start 80.5 85) (end 84 81.5) (width 0.2) (layer "F.Cu") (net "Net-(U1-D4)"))
 (segment (start 80.5 75.5) (end 84 79) (width 0.2) (layer "F.Cu") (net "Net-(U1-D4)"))
 (segment (start 74.4 57.83) (end 80.5 63.93) (width 0.2) (layer "F.Cu") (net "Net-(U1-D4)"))
 (segment (start 84 81.5) (end 84 79) (width 0.2) (layer "F.Cu") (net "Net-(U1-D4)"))
 (via (at 84 79) (size 0.6) (drill 0.3) (layers "F.Cu" "B.Cu") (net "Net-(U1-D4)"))
 (via (at 80.5 85) (size 0.6) (drill 0.3) (layers "F.Cu" "B.Cu") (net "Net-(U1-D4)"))
 (segment (start 79.42 99.5) (end 79.42 97.58) (width 0.2) (layer "B.Cu") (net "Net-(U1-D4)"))
 (segment (start 80.5 96.5) (end 80.5 85) (width 0.2) (layer "B.Cu") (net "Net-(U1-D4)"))
 (segment (start 86 81) (end 86 85) (width 0.2) (layer "B.Cu") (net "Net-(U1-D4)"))
 (segment (start 79.42 97.58) (end 80.5 96.5) (width 0.2) (layer "B.Cu") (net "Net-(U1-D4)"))
 (segment (start 84 79) (end 86 81) (width 0.2) (layer "B.Cu") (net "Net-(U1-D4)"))
 (segment (start 74.4 114.83) (end 74.4 113.4) (width 0.2) (layer "F.Cu") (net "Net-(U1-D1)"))
 (segment (start 74.4 113.4) (end 73 112) (width 0.2) (layer "F.Cu") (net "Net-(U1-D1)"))
 (via (at 73 112) (size 0.6) (drill 0.3) (layers "F.Cu" "B.Cu") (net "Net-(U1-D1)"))
 (segment (start 73 112) (end 78.5 112) (width 0.2) (layer "B.Cu") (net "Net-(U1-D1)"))
 (segment (start 81.660001 104.749999) (end 81.96 104.45) (width 0.2) (layer "B.Cu") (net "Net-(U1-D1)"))
 (segment (start 81.660001 108.839999) (end 81.660001 104.749999) (width 0.2) (layer "B.Cu") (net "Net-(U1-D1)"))
 (segment (start 78.5 112) (end 81.660001 108.839999) (width 0.2) (layer "B.Cu") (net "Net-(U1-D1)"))
 (segment (start 69.5 111.9125) (end 72.9125 111.9125) (width 0.2) (layer "B.Cu") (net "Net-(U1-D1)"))
 (segment (start 72.9125 111.9125) (end 73 112) (width 0.2) (layer "B.Cu") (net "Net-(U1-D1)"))
 (segment (start 81.7 123.424501) (end 83.9 121.224501) (width 0.2) (layer "F.Cu") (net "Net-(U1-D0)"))
 (segment (start 77.45 130.85) (end 78.680509 130.85) (width 0.2) (layer "F.Cu") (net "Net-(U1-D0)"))
 (segment (start 83.9 121.224501) (end 83.9 116.424265) (width 0.2) (layer "F.Cu") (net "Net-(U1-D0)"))
 (segment (start 81.7 127.830509) (end 81.7 123.424501) (width 0.2) (layer "F.Cu") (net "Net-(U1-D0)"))
 (segment (start 78.680509 130.85) (end 81.7 127.830509) (width 0.2) (layer "F.Cu") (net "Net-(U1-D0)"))
 (segment (start 83.9 116.424265) (end 84.004265 116.32) (width 0.2) (layer "F.Cu") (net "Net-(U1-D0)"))
 (segment (start 74.4 133.9) (end 77.45 130.85) (width 0.2) (layer "F.Cu") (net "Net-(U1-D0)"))
 (via (at 84.004265 116.32) (size 0.6) (drill 0.3) (layers "F.Cu" "B.Cu") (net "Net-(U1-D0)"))
 (segment (start 83.23 106.1425) (end 86 108.9125) (width 0.2) (layer "B.Cu") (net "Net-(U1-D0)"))
 (segment (start 86 114.324265) (end 86 108.9125) (width 0.2) (layer "B.Cu") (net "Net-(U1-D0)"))
 (segment (start 84.004265 116.32) (end 86 114.324265) (width 0.2) (layer "B.Cu") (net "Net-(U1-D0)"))
 (segment (start 83.23 104.45) (end 83.23 106.1425) (width 0.2) (layer "B.Cu") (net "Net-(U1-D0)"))
 (segment (start 74.748529 106.1) (end 71.1 106.1) (width 0.2) (layer "F.Cu") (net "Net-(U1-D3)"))
 (segment (start 71 106) (end 71 91.5) (width 0.2) (layer "F.Cu") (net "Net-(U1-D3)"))
 (segment (start 70.17 76.83) (end 74.4 76.83) (width 0.2) (layer "F.Cu") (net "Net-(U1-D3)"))
 (segment (start 71.1 106.1) (end 71 106) (width 0.2) (layer "F.Cu") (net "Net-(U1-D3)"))
 (segment (start 69.5 83) (end 69.5 77.5) (width 0.2) (layer "F.Cu") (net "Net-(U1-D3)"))
 (segment (start 74.848529 106) (end 74.748529 106.1) (width 0.2) (layer "F.Cu") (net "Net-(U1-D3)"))
 (segment (start 69.5 77.5) (end 70.17 76.83) (width 0.2) (layer "F.Cu") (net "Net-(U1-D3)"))
 (segment (start 79.5 106) (end 74.848529 106) (width 0.2) (layer "F.Cu") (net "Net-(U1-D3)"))
 (via (at 71 91.5) (size 0.6) (drill 0.3) (layers "F.Cu" "B.Cu") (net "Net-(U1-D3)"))
 (via (at 69.5 83) (size 0.6) (drill 0.3) (layers "F.Cu" "B.Cu") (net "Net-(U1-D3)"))
 (via (at 79.5 106) (size 0.6) (drill 0.3) (layers "F.Cu" "B.Cu") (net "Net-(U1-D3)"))
 (segment (start 79.42 104.45) (end 79.42 105.92) (width 0.2) (layer "B.Cu") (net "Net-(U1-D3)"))
 (segment (start 70.4125 91.5) (end 69.5 90.5875) (width 0.2) (layer "B.Cu") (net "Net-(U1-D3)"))
 (segment (start 79.42 105.92) (end 79.5 106) (width 0.2) (layer "B.Cu") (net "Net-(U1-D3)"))
 (segment (start 69.5 90.5875) (end 69.5 83) (width 0.2) (layer "B.Cu") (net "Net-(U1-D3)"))
 (segment (start 71 91.5) (end 70.4125 91.5) (width 0.2) (layer "B.Cu") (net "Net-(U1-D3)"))
 (segment (start 74.4 95.76) (end 74.4 105.4) (width 0.2) (layer "F.Cu") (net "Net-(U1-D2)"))
 (segment (start 74.4 105.4) (end 74.5 105.5) (width 0.2) (layer "F.Cu") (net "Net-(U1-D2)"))
 (via (at 74.5 105.5) (size 0.6) (drill 0.3) (layers "F.Cu" "B.Cu") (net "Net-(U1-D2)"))
 (segment (start 70.4125 103.851688) (end 70.4125 103.5) (width 0.2) (layer "B.Cu") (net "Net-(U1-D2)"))
 (segment (start 74.5 104.5) (end 74.5 105.5) (width 0.2) (layer "B.Cu") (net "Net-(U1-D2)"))
 (segment (start 72.060812 105.5) (end 70.4125 103.851688) (width 0.2) (layer "B.Cu") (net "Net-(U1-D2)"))
 (segment (start 77 102) (end 74.5 104.5) (width 0.2) (layer "B.Cu") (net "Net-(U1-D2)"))
 (segment (start 80.69 104.45) (end 80.69 102.19) (width 0.2) (layer "B.Cu") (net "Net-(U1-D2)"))
 (segment (start 80.69 102.19) (end 80.5 102) (width 0.2) (layer "B.Cu") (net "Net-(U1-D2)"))
 (segment (start 74.5 105.5) (end 72.060812 105.5) (width 0.2) (layer "B.Cu") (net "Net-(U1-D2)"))
 (segment (start 70.4125 103.5) (end 69.5 102.5875) (width 0.2) (layer "B.Cu") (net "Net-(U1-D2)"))
 (segment (start 80.5 102) (end 77 102) (width 0.2) (layer "B.Cu") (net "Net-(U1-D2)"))
 (segment (start 83.538478 110.23) (end 84.5 109.268478) (width 0.2) (layer "F.Cu") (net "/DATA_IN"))
 (segment (start 82.283705 110.23) (end 83.538478 110.23) (width 0.2) (layer "F.Cu") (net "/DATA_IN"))
 (segment (start 84.5 109.268478) (end 84.5 106) (width 0.2) (layer "F.Cu") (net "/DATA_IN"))
 (segment (start 80.5 112.013705) (end 82.283705 110.23) (width 0.2) (layer "F.Cu") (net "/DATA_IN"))
 (segment (start 82 121.5) (end 80.5 120) (width 0.2) (layer "F.Cu") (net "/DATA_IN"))
 (segment (start 80.5 120) (end 80.5 112.013705) (width 0.2) (layer "F.Cu") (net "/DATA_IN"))
 (via (at 84.5 106) (size 0.6) (drill 0.3) (layers "F.Cu" "B.Cu") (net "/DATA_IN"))
 (via (at 82 121.5) (size 0.6) (drill 0.3) (layers "F.Cu" "B.Cu") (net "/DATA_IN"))
 (segment (start 69 127.12) (end 69 125.5) (width 0.2) (layer "B.Cu") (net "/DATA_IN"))
 (segment (start 71.15 123.35) (end 71.15 122.040812) (width 0.2) (layer "B.Cu") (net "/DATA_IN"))
 (segment (start 84.5 106) (end 84.5 104.45) (width 0.2) (layer "B.Cu") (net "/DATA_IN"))
 (segment (start 71.15 122.040812) (end 71.940812 121.25) (width 0.2) (layer "B.Cu") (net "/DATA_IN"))
 (segment (start 71.940812 121.25) (end 81.75 121.25) (width 0.2) (layer "B.Cu") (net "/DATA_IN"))
 (segment (start 81.75 121.25) (end 82 121.5) (width 0.2) (layer "B.Cu") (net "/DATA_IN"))
 (segment (start 69 125.5) (end 71.15 123.35) (width 0.2) (layer "B.Cu") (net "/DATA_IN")))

